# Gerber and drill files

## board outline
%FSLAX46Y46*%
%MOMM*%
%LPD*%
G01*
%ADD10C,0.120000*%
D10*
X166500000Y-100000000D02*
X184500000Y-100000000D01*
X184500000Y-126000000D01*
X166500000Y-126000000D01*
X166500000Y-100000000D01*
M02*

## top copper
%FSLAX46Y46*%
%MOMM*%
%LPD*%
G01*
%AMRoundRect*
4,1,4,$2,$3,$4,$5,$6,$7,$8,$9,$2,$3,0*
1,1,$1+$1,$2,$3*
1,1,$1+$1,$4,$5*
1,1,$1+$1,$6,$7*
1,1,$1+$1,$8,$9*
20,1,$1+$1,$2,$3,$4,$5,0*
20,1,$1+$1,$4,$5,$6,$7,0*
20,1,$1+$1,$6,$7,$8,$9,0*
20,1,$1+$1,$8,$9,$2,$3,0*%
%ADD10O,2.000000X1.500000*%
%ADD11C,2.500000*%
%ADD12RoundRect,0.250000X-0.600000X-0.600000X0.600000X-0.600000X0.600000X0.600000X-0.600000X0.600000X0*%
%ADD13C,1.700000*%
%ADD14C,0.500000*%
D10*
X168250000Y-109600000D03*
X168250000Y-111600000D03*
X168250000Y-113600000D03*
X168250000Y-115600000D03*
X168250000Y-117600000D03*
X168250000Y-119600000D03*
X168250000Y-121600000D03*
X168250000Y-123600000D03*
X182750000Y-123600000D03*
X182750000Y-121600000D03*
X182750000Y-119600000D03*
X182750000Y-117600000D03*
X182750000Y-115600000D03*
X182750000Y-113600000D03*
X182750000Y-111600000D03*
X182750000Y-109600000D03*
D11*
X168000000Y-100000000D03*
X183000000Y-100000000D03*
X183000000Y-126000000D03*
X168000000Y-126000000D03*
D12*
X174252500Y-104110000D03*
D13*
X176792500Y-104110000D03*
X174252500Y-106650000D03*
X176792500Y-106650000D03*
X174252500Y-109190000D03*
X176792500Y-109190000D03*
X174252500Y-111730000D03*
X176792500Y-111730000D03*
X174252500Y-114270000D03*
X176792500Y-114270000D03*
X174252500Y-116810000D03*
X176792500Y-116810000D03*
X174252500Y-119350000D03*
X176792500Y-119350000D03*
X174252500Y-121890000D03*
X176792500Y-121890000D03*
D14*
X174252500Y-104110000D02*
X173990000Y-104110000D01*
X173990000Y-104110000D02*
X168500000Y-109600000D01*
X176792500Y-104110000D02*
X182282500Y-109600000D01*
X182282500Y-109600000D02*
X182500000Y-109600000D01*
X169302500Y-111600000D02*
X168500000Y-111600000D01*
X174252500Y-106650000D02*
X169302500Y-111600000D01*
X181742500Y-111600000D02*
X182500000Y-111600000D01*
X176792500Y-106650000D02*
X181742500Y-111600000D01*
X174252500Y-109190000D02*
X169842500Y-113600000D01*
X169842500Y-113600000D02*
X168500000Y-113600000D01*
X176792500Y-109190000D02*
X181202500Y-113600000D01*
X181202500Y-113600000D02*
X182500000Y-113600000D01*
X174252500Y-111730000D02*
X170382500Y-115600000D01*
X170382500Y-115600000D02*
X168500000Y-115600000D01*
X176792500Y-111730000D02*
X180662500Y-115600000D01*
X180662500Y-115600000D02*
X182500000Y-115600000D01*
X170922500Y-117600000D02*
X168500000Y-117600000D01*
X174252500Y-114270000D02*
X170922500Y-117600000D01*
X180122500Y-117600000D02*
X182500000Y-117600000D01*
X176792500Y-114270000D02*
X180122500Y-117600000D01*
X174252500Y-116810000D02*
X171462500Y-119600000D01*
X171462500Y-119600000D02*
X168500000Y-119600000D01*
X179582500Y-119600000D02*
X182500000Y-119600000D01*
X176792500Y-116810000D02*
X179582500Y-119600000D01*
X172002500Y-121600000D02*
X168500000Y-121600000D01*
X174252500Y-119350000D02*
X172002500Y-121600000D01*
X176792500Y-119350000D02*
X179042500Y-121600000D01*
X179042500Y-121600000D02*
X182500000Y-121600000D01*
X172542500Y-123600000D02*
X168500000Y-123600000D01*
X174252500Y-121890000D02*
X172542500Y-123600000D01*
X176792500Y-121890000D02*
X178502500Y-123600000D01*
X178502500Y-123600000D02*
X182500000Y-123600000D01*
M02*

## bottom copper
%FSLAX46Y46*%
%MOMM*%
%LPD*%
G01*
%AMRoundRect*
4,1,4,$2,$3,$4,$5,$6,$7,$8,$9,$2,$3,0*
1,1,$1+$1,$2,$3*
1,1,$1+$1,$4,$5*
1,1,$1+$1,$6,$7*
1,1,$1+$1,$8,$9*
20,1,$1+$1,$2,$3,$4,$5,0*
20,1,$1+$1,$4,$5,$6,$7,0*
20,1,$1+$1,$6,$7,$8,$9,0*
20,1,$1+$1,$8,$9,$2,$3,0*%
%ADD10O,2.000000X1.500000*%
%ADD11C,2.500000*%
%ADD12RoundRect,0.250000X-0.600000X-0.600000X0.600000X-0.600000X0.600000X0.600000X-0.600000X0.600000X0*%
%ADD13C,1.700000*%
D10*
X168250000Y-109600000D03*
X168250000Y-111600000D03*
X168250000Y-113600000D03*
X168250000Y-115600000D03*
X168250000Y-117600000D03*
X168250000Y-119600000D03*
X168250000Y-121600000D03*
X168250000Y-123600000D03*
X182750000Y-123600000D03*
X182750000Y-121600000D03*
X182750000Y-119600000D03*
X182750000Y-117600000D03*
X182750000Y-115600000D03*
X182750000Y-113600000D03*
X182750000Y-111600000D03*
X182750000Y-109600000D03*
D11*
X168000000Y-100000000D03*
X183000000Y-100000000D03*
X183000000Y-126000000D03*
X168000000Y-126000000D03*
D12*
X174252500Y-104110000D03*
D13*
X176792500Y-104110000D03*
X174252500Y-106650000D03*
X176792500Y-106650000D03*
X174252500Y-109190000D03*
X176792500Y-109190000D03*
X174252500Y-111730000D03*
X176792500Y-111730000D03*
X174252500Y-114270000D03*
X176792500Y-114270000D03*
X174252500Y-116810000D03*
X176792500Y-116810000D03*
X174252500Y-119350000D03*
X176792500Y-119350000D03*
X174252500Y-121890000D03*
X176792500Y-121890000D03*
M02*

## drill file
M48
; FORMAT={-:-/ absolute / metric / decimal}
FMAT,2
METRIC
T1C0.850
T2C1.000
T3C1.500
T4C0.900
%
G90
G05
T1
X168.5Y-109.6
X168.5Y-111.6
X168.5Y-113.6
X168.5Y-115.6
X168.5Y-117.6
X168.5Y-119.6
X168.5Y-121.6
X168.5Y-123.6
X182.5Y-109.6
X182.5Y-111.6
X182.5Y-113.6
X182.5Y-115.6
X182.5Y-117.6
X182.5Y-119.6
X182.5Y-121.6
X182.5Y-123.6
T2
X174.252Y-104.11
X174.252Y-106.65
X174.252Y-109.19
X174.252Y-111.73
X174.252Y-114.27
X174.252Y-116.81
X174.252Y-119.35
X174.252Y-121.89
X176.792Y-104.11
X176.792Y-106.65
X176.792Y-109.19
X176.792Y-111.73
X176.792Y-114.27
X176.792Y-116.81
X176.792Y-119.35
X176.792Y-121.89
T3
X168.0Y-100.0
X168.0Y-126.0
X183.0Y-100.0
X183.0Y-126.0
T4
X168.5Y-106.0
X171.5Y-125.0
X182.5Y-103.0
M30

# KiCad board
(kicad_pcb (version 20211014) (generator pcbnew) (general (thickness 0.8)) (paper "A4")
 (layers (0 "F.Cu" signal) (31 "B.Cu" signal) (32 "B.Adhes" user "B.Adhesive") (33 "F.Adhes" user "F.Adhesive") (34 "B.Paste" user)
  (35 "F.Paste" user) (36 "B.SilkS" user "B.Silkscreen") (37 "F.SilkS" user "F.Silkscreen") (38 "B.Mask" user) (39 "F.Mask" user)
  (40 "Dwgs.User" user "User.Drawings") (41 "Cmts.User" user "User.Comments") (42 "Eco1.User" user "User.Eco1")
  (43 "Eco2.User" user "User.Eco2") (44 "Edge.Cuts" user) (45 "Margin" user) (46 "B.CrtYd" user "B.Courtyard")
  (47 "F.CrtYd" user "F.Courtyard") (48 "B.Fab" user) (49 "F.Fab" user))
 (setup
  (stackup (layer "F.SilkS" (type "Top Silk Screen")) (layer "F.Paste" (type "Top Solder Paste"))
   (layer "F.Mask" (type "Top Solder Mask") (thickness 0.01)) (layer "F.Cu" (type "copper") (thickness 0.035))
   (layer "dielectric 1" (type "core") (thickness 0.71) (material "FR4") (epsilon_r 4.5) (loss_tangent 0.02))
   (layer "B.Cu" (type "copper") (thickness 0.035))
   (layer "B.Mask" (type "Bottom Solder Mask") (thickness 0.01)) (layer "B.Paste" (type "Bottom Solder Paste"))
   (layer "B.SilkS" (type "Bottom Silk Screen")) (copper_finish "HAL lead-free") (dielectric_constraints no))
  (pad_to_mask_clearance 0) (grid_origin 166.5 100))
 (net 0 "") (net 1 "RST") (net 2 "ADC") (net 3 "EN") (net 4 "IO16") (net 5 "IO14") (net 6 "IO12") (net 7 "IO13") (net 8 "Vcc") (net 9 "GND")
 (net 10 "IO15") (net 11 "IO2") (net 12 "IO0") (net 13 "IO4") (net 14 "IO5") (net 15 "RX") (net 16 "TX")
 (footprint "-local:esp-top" (layer "F.Cu") (at 166.5 100)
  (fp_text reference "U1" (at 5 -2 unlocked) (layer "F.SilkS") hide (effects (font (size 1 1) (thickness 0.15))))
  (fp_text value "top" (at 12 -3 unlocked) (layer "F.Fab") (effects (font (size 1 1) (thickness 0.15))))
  (pad "1" thru_hole oval (at 2 9.6) (size 2 1.5) (drill 0.85 (offset -0.25 0)) (layers *.Cu *.Mask) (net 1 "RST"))
  (pad "2" thru_hole oval (at 2 11.6) (size 2 1.5) (drill 0.85 (offset -0.25 0)) (layers *.Cu *.Mask) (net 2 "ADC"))
  (pad "3" thru_hole oval (at 2 13.6) (size 2 1.5) (drill 0.85 (offset -0.25 0)) (layers *.Cu *.Mask) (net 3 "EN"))
  (pad "4" thru_hole oval (at 2 15.6) (size 2 1.5) (drill 0.85 (offset -0.25 0)) (layers *.Cu *.Mask) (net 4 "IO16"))
  (pad "5" thru_hole oval (at 2 17.6) (size 2 1.5) (drill 0.85 (offset -0.25 0)) (layers *.Cu *.Mask) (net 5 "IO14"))
  (pad "6" thru_hole oval (at 2 19.6) (size 2 1.5) (drill 0.85 (offset -0.25 0)) (layers *.Cu *.Mask) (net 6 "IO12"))
  (pad "7" thru_hole oval (at 2 21.6) (size 2 1.5) (drill 0.85 (offset -0.25 0)) (layers *.Cu *.Mask) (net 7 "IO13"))
  (pad "8" thru_hole oval (at 2 23.6) (size 2 1.5) (drill 0.85 (offset -0.25 0)) (layers *.Cu *.Mask) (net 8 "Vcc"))
  (pad "9" thru_hole oval (at 16 23.6 180) (size 2 1.5) (drill 0.85 (offset -0.25 0)) (layers *.Cu *.Mask) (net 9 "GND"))
  (pad "10" thru_hole oval (at 16 21.6 180) (size 2 1.5) (drill 0.85 (offset -0.25 0)) (layers *.Cu *.Mask) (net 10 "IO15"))
  (pad "11" thru_hole oval (at 16 19.6 180) (size 2 1.5) (drill 0.85 (offset -0.25 0)) (layers *.Cu *.Mask) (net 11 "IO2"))
  (pad "12" thru_hole oval (at 16 17.6 180) (size 2 1.5) (drill 0.85 (offset -0.25 0)) (layers *.Cu *.Mask) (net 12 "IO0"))
  (pad "13" thru_hole oval (at 16 15.6 180) (size 2 1.5) (drill 0.85 (offset -0.25 0)) (layers *.Cu *.Mask) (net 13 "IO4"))
  (pad "14" thru_hole oval (at 16 13.6 180) (size 2 1.5) (drill 0.85 (offset -0.25 0)) (layers *.Cu *.Mask) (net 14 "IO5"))
  (pad "15" thru_hole oval (at 16 11.6 180) (size 2 1.5) (drill 0.85 (offset -0.25 0)) (layers *.Cu *.Mask) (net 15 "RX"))
  (pad "16" thru_hole oval (at 16 9.6 180) (size 2 1.5) (drill 0.85 (offset -0.25 0)) (layers *.Cu *.Mask) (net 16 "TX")))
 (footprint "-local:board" (layer "F.Cu") (at 166.5 100)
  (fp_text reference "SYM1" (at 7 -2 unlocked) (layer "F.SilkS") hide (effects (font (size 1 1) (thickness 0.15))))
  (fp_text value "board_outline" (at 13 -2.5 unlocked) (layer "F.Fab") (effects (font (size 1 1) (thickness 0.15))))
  (fp_rect (start 0 0) (end 18 26) (layer "Edge.Cuts") (width 0.12) (fill none))
  (pad "" np_thru_hole circle (at 16 3) (size 0.9 0.9) (drill 0.9) (layers F&B.Cu *.Mask))
  (pad "" np_thru_hole circle (at 5 25) (size 0.9 0.9) (drill 0.9) (layers F&B.Cu *.Mask))
  (pad "" np_thru_hole circle (at 2 6) (size 0.9 0.9) (drill 0.9) (layers F&B.Cu *.Mask))
  (pad "1" thru_hole circle (at 1.5 0) (size 2.5 2.5) (drill 1.5) (layers *.Cu *.Mask))
  (pad "2" thru_hole circle (at 16.5 0) (size 2.5 2.5) (drill 1.5) (layers *.Cu *.Mask))
  (pad "3" thru_hole circle (at 16.5 26) (size 2.5 2.5) (drill 1.5) (layers *.Cu *.Mask))
  (pad "4" thru_hole circle (at 1.5 26) (size 2.5 2.5) (drill 1.5) (layers *.Cu *.Mask)))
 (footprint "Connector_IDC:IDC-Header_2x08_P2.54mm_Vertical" (layer "F.Cu") (at 174.2525 104.11)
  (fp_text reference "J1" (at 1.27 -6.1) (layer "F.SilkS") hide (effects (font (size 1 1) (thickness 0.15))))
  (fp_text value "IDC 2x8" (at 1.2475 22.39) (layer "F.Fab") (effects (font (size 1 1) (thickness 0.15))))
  (pad "1" thru_hole roundrect (at 0 0) (size 1.7 1.7) (drill 1) (layers *.Cu *.Mask) (roundrect_rratio 0.147059) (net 1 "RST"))
  (pad "2" thru_hole circle (at 2.54 0) (size 1.7 1.7) (drill 1) (layers *.Cu *.Mask) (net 16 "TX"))
  (pad "3" thru_hole circle (at 0 2.54) (size 1.7 1.7) (drill 1) (layers *.Cu *.Mask) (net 2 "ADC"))
  (pad "4" thru_hole circle (at 2.54 2.54) (size 1.7 1.7) (drill 1) (layers *.Cu *.Mask) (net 15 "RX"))
  (pad "5" thru_hole circle (at 0 5.08) (size 1.7 1.7) (drill 1) (layers *.Cu *.Mask) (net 3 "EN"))
  (pad "6" thru_hole circle (at 2.54 5.08) (size 1.7 1.7) (drill 1) (layers *.Cu *.Mask) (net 14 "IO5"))
  (pad "7" thru_hole circle (at 0 7.62) (size 1.7 1.7) (drill 1) (layers *.Cu *.Mask) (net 4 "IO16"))
  (pad "8" thru_hole circle (at 2.54 7.62) (size 1.7 1.7) (drill 1) (layers *.Cu *.Mask) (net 13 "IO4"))
  (pad "9" thru_hole circle (at 0 10.16) (size 1.7 1.7) (drill 1) (layers *.Cu *.Mask) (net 5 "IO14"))
  (pad "10" thru_hole circle (at 2.54 10.16) (size 1.7 1.7) (drill 1) (layers *.Cu *.Mask) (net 12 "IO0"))
  (pad "11" thru_hole circle (at 0 12.7) (size 1.7 1.7) (drill 1) (layers *.Cu *.Mask) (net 6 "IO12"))
  (pad "12" thru_hole circle (at 2.54 12.7) (size 1.7 1.7) (drill 1) (layers *.Cu *.Mask) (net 11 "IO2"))
  (pad "13" thru_hole circle (at 0 15.24) (size 1.7 1.7) (drill 1) (layers *.Cu *.Mask) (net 7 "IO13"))
  (pad "14" thru_hole circle (at 2.54 15.24) (size 1.7 1.7) (drill 1) (layers *.Cu *.Mask) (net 10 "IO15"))
  (pad "15" thru_hole circle (at 0 17.78) (size 1.7 1.7) (drill 1) (layers *.Cu *.Mask) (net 8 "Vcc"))
  (pad "16" thru_hole circle (at 2.54 17.78) (size 1.7 1.7) (drill 1) (layers *.Cu *.Mask) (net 9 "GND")))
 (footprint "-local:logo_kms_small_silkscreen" (layer "B.Cu") (at 181.7 105.4 180)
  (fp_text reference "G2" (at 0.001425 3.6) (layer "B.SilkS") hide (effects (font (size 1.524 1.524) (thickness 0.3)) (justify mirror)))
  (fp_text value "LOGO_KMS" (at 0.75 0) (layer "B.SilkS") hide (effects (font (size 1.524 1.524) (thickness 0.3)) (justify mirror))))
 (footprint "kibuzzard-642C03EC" (layer "B.Cu") (at 175.5 124.2 180)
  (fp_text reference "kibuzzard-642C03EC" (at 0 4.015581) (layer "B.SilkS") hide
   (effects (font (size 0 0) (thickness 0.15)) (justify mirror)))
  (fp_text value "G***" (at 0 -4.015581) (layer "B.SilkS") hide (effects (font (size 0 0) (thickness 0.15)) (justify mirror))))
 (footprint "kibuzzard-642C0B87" (layer "B.Cu") (at 170.5 112.6 90)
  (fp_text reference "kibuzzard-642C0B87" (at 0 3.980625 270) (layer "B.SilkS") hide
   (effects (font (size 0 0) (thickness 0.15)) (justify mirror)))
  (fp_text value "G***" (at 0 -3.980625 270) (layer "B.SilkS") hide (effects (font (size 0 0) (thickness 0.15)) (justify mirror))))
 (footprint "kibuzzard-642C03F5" (layer "B.Cu") (at 175.5 101.6 180)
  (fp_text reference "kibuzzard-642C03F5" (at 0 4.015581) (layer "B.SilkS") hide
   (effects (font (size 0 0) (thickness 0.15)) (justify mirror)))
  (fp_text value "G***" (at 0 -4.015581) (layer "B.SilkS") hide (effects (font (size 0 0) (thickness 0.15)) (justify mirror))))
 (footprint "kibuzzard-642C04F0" (layer "B.Cu") (at 180.1 116 -90)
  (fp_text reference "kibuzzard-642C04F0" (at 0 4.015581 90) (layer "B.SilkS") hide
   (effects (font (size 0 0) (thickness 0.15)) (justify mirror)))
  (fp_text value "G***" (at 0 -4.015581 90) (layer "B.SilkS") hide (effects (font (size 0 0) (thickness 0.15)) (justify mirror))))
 (segment (start 174.2525 104.11) (end 173.99 104.11) (width 0.5) (layer "F.Cu") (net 1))
 (segment (start 173.99 104.11) (end 168.5 109.6) (width 0.5) (layer "F.Cu") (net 1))
 (segment (start 176.7925 104.11) (end 182.2825 109.6) (width 0.5) (layer "F.Cu") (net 16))
 (segment (start 182.2825 109.6) (end 182.5 109.6) (width 0.5) (layer "F.Cu") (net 16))
 (segment (start 169.3025 111.6) (end 168.5 111.6) (width 0.5) (layer "F.Cu") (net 2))
 (segment (start 174.2525 106.65) (end 169.3025 111.6) (width 0.5) (layer "F.Cu") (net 2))
 (segment (start 181.7425 111.6) (end 182.5 111.6) (width 0.5) (layer "F.Cu") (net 15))
 (segment (start 176.7925 106.65) (end 181.7425 111.6) (width 0.5) (layer "F.Cu") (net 15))
 (segment (start 174.2525 109.19) (end 169.8425 113.6) (width 0.5) (layer "F.Cu") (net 3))
 (segment (start 169.8425 113.6) (end 168.5 113.6) (width 0.5) (layer "F.Cu") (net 3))
 (segment (start 176.7925 109.19) (end 181.2025 113.6) (width 0.5) (layer "F.Cu") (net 14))
 (segment (start 181.2025 113.6) (end 182.5 113.6) (width 0.5) (layer "F.Cu") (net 14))
 (segment (start 174.2525 111.73) (end 170.3825 115.6) (width 0.5) (layer "F.Cu") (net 4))
 (segment (start 170.3825 115.6) (end 168.5 115.6) (width 0.5) (layer "F.Cu") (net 4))
 (segment (start 176.7925 111.73) (end 180.6625 115.6) (width 0.5) (layer "F.Cu") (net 13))
 (segment (start 180.6625 115.6) (end 182.5 115.6) (width 0.5) (layer "F.Cu") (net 13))
 (segment (start 170.9225 117.6) (end 168.5 117.6) (width 0.5) (layer "F.Cu") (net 5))
 (segment (start 174.2525 114.27) (end 170.9225 117.6) (width 0.5) (layer "F.Cu") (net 5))
 (segment (start 180.1225 117.6) (end 182.5 117.6) (width 0.5) (layer "F.Cu") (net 12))
 (segment (start 176.7925 114.27) (end 180.1225 117.6) (width 0.5) (layer "F.Cu") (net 12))
 (segment (start 174.2525 116.81) (end 171.4625 119.6) (width 0.5) (layer "F.Cu") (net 6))
 (segment (start 171.4625 119.6) (end 168.5 119.6) (width 0.5) (layer "F.Cu") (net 6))
 (segment (start 179.5825 119.6) (end 182.5 119.6) (width 0.5) (layer "F.Cu") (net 11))
 (segment (start 176.7925 116.81) (end 179.5825 119.6) (width 0.5) (layer "F.Cu") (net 11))
 (segment (start 172.0025 121.6) (end 168.5 121.6) (width 0.5) (layer "F.Cu") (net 7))
 (segment (start 174.2525 119.35) (end 172.0025 121.6) (width 0.5) (layer "F.Cu") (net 7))
 (segment (start 176.7925 119.35) (end 179.0425 121.6) (width 0.5) (layer "F.Cu") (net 10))
 (segment (start 179.0425 121.6) (end 182.5 121.6) (width 0.5) (layer "F.Cu") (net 10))
 (segment (start 172.5425 123.6) (end 168.5 123.6) (width 0.5) (layer "F.Cu") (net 8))
 (segment (start 174.2525 121.89) (end 172.5425 123.6) (width 0.5) (layer "F.Cu") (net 8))
 (segment (start 176.7925 121.89) (end 178.5025 123.6) (width 0.5) (layer "F.Cu") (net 9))
 (segment (start 178.5025 123.6) (end 182.5 123.6) (width 0.5) (layer "F.Cu") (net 9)))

